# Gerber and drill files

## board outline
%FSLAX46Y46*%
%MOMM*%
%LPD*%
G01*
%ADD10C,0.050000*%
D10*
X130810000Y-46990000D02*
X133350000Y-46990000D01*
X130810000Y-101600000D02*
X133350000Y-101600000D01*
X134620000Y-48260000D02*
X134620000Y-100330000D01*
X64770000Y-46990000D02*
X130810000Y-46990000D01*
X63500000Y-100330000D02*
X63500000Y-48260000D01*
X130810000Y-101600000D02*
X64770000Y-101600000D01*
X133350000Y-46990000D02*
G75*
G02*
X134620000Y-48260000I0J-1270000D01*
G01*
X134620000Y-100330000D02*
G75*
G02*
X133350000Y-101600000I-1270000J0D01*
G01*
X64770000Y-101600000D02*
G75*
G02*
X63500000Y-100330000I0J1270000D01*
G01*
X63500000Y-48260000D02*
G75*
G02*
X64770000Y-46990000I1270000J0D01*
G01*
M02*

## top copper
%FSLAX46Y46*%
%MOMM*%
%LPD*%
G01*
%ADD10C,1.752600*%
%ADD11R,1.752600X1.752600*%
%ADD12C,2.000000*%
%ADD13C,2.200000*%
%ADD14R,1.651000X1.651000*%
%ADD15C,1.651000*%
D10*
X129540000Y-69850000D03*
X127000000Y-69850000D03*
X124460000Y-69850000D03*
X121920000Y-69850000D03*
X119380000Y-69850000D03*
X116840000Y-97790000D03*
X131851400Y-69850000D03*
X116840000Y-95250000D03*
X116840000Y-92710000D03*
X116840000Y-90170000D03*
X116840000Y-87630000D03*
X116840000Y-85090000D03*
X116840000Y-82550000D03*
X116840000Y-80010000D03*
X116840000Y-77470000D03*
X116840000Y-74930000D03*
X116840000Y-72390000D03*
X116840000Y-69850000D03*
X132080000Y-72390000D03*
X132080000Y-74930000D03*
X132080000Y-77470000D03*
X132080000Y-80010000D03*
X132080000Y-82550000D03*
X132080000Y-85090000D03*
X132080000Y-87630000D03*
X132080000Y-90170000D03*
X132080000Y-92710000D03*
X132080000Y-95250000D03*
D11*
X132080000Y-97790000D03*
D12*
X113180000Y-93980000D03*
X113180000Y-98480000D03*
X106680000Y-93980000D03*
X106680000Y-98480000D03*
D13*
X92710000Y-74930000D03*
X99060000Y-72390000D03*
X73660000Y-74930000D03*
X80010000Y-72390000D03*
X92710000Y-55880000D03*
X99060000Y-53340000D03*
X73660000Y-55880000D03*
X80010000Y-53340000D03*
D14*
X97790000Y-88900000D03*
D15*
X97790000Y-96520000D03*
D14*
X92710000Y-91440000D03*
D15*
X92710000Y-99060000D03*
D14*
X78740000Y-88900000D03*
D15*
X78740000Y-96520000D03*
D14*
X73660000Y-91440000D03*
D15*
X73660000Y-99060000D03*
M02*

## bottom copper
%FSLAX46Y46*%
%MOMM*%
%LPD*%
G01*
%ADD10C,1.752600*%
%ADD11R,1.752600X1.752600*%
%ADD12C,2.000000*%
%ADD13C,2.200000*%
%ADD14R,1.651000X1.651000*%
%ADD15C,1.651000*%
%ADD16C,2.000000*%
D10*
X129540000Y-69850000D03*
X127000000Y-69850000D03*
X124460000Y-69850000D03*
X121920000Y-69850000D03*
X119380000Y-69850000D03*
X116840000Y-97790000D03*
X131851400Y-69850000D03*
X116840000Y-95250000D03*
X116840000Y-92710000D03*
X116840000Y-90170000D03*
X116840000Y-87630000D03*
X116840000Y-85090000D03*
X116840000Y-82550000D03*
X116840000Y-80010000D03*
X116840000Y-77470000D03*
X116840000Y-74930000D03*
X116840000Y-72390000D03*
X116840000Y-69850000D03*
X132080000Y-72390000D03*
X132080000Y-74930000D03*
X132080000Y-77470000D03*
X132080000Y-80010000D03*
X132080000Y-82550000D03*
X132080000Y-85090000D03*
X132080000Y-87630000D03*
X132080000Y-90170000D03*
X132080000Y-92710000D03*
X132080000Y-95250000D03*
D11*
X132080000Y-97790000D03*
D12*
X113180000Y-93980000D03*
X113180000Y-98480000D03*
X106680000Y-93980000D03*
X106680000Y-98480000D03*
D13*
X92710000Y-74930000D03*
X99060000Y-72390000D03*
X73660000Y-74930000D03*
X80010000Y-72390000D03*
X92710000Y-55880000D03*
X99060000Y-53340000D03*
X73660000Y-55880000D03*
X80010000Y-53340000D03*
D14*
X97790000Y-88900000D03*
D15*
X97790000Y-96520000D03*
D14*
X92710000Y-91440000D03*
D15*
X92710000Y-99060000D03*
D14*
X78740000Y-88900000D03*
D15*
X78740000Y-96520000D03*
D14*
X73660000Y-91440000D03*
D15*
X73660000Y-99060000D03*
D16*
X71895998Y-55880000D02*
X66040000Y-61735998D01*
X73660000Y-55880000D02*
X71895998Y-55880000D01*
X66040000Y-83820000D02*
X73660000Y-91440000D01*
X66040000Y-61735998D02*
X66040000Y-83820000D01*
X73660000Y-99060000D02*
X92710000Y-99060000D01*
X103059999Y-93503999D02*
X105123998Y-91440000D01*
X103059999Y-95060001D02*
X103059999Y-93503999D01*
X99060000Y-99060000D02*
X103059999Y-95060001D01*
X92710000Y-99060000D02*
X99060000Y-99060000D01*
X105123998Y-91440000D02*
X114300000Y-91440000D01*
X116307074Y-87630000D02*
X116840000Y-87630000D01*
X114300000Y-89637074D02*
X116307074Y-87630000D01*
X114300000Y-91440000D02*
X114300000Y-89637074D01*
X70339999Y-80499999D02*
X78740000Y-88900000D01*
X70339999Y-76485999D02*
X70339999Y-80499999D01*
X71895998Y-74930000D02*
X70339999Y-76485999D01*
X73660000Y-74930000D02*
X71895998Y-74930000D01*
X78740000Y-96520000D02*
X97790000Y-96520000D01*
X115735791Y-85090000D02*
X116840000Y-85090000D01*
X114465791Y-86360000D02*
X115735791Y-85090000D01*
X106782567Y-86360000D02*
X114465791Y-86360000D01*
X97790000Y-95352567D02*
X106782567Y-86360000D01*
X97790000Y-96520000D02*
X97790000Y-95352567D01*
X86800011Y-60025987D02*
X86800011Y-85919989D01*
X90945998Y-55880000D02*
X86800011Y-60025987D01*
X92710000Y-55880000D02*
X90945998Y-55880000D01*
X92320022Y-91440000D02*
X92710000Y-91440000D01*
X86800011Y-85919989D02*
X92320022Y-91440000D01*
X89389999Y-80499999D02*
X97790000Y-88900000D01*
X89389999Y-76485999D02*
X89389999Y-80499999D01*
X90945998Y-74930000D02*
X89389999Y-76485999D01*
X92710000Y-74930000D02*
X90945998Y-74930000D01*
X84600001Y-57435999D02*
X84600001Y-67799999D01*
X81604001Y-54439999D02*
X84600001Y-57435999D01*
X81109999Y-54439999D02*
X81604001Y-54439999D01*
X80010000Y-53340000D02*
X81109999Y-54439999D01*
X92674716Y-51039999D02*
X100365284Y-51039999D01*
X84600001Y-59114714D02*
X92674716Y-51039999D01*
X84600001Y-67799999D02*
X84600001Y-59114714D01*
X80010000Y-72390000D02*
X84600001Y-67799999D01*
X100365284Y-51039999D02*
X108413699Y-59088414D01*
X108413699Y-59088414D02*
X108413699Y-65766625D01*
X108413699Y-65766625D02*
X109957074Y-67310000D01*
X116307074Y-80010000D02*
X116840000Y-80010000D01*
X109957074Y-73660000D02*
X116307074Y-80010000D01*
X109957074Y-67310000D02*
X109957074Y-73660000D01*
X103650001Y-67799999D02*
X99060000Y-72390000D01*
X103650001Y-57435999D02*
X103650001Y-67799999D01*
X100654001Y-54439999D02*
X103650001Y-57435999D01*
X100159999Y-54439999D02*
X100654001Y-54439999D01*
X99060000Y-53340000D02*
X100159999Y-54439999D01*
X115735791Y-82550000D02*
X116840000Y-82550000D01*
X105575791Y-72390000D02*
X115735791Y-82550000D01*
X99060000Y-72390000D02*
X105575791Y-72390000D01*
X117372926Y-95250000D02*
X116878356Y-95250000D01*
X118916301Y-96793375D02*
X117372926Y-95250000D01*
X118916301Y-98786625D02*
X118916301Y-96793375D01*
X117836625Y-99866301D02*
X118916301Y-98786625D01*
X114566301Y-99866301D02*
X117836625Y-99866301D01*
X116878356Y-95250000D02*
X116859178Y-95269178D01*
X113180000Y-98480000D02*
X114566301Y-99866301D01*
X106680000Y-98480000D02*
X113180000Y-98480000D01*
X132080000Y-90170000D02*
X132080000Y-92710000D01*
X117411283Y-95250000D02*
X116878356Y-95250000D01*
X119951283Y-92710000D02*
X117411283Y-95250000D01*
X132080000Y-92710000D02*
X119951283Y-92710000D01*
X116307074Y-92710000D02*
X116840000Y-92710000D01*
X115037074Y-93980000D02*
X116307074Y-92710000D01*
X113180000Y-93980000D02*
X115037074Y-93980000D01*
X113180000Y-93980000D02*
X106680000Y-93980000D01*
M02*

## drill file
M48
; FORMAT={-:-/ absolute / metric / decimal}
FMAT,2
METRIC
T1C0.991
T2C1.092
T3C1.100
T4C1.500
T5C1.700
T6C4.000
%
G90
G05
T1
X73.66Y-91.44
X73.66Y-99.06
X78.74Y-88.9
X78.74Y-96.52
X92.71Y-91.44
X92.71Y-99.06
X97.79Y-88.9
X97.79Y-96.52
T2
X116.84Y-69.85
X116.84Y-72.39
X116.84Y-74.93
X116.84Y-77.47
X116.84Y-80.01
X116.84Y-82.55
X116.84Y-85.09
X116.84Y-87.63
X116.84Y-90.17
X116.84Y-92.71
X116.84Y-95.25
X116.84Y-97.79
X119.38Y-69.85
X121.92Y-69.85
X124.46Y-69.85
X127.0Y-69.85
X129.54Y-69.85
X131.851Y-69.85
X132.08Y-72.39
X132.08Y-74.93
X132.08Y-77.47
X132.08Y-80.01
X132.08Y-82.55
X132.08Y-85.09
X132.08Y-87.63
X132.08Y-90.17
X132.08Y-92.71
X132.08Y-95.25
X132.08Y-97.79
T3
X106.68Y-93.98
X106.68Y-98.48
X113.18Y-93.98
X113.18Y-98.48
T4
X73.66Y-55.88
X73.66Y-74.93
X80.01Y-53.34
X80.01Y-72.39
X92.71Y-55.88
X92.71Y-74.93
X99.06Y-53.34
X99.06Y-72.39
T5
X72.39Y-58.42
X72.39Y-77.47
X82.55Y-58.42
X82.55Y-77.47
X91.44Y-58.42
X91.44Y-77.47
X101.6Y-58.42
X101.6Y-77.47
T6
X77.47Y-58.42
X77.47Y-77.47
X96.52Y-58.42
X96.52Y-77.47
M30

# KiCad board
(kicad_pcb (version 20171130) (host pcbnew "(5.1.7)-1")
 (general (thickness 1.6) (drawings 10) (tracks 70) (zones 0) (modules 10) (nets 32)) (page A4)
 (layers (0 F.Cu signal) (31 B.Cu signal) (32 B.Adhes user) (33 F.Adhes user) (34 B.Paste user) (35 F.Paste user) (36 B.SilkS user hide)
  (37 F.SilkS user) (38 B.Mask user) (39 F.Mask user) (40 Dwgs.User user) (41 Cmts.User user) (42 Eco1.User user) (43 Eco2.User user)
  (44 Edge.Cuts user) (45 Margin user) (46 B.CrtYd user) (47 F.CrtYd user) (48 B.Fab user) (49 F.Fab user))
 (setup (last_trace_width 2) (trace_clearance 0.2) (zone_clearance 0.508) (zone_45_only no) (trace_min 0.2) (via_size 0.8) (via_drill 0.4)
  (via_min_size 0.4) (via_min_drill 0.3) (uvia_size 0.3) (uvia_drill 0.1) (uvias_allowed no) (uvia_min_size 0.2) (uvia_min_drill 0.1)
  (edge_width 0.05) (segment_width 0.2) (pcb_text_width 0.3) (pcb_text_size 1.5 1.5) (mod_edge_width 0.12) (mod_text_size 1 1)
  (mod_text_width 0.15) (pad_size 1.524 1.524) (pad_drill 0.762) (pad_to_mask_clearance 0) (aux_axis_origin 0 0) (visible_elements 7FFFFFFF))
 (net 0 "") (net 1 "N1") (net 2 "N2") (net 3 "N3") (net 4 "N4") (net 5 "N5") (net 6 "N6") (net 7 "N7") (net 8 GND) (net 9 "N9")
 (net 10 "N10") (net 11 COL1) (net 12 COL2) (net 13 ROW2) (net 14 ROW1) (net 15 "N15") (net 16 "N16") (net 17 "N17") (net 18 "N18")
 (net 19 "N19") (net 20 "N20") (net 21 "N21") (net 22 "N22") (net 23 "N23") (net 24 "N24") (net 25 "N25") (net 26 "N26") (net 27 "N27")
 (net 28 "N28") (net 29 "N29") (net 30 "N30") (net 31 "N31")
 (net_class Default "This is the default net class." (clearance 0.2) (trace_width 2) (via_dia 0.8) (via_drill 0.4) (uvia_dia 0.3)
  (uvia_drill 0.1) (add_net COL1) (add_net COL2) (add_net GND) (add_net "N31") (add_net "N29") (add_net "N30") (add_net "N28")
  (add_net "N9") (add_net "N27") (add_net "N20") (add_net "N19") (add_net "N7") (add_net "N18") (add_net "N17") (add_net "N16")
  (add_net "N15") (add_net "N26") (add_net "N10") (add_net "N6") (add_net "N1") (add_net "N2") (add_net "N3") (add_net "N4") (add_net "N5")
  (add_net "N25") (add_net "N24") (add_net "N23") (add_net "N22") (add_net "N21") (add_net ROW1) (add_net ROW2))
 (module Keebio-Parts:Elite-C (layer F.Cu) (at 124.46 83.82 90)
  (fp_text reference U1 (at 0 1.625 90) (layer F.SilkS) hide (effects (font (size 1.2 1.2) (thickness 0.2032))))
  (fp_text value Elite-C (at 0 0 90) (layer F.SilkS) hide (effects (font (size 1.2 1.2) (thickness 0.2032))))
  (pad 25 thru_hole circle (at 13.97 5.08 90) (size 1.7526 1.7526) (drill 1.0922) (layers *.Cu *.SilkS *.Mask) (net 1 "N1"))
  (pad 26 thru_hole circle (at 13.97 2.54 90) (size 1.7526 1.7526) (drill 1.0922) (layers *.Cu *.SilkS *.Mask) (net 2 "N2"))
  (pad 27 thru_hole circle (at 13.97 0 90) (size 1.7526 1.7526) (drill 1.0922) (layers *.Cu *.SilkS *.Mask) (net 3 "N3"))
  (pad 28 thru_hole circle (at 13.97 -2.54 90) (size 1.7526 1.7526) (drill 1.0922) (layers *.Cu *.SilkS *.Mask) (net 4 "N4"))
  (pad 29 thru_hole circle (at 13.97 -5.08 90) (size 1.7526 1.7526) (drill 1.0922) (layers *.Cu *.SilkS *.Mask) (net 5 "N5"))
  (pad 24 thru_hole circle (at -13.97 -7.62 90) (size 1.7526 1.7526) (drill 1.0922) (layers *.Cu *.SilkS *.Mask) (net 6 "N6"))
  (pad 12 thru_hole circle (at 13.97 7.3914 90) (size 1.7526 1.7526) (drill 1.0922) (layers *.Cu *.SilkS *.Mask) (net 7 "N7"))
  (pad 23 thru_hole circle (at -11.43 -7.62 90) (size 1.7526 1.7526) (drill 1.0922) (layers *.Cu *.SilkS *.Mask) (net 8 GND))
  (pad 22 thru_hole circle (at -8.89 -7.62 90) (size 1.7526 1.7526) (drill 1.0922) (layers *.Cu *.SilkS *.Mask) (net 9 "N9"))
  (pad 21 thru_hole circle (at -6.35 -7.62 90) (size 1.7526 1.7526) (drill 1.0922) (layers *.Cu *.SilkS *.Mask) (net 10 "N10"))
  (pad 20 thru_hole circle (at -3.81 -7.62 90) (size 1.7526 1.7526) (drill 1.0922) (layers *.Cu *.SilkS *.Mask) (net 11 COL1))
  (pad 19 thru_hole circle (at -1.27 -7.62 90) (size 1.7526 1.7526) (drill 1.0922) (layers *.Cu *.SilkS *.Mask) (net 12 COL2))
  (pad 18 thru_hole circle (at 1.27 -7.62 90) (size 1.7526 1.7526) (drill 1.0922) (layers *.Cu *.SilkS *.Mask) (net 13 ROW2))
  (pad 17 thru_hole circle (at 3.81 -7.62 90) (size 1.7526 1.7526) (drill 1.0922) (layers *.Cu *.SilkS *.Mask) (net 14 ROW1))
  (pad 16 thru_hole circle (at 6.35 -7.62 90) (size 1.7526 1.7526) (drill 1.0922) (layers *.Cu *.SilkS *.Mask) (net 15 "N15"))
  (pad 15 thru_hole circle (at 8.89 -7.62 90) (size 1.7526 1.7526) (drill 1.0922) (layers *.Cu *.SilkS *.Mask) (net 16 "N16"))
  (pad 14 thru_hole circle (at 11.43 -7.62 90) (size 1.7526 1.7526) (drill 1.0922) (layers *.Cu *.SilkS *.Mask) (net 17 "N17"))
  (pad 13 thru_hole circle (at 13.97 -7.62 90) (size 1.7526 1.7526) (drill 1.0922) (layers *.Cu *.SilkS *.Mask) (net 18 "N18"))
  (pad 11 thru_hole circle (at 11.43 7.62 90) (size 1.7526 1.7526) (drill 1.0922) (layers *.Cu *.SilkS *.Mask) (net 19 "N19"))
  (pad 10 thru_hole circle (at 8.89 7.62 90) (size 1.7526 1.7526) (drill 1.0922) (layers *.Cu *.SilkS *.Mask) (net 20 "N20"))
  (pad 9 thru_hole circle (at 6.35 7.62 90) (size 1.7526 1.7526) (drill 1.0922) (layers *.Cu *.SilkS *.Mask) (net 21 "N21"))
  (pad 8 thru_hole circle (at 3.81 7.62 90) (size 1.7526 1.7526) (drill 1.0922) (layers *.Cu *.SilkS *.Mask) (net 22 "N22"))
  (pad 7 thru_hole circle (at 1.27 7.62 90) (size 1.7526 1.7526) (drill 1.0922) (layers *.Cu *.SilkS *.Mask) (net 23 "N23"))
  (pad 6 thru_hole circle (at -1.27 7.62 90) (size 1.7526 1.7526) (drill 1.0922) (layers *.Cu *.SilkS *.Mask) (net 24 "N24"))
  (pad 5 thru_hole circle (at -3.81 7.62 90) (size 1.7526 1.7526) (drill 1.0922) (layers *.Cu *.SilkS *.Mask) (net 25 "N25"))
  (pad 4 thru_hole circle (at -6.35 7.62 90) (size 1.7526 1.7526) (drill 1.0922) (layers *.Cu *.SilkS *.Mask) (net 8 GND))
  (pad 3 thru_hole circle (at -8.89 7.62 90) (size 1.7526 1.7526) (drill 1.0922) (layers *.Cu *.SilkS *.Mask) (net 8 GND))
  (pad 2 thru_hole circle (at -11.43 7.62 90) (size 1.7526 1.7526) (drill 1.0922) (layers *.Cu *.SilkS *.Mask) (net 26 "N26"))
  (pad 1 thru_hole rect (at -13.97 7.62 90) (size 1.7526 1.7526) (drill 1.0922) (layers *.Cu *.SilkS *.Mask) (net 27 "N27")))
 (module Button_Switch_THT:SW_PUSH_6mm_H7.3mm (layer F.Cu) (at 106.68 93.98)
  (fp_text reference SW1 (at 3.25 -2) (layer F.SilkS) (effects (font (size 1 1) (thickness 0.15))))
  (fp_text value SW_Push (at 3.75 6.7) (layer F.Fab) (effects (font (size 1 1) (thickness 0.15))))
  (pad 1 thru_hole circle (at 6.5 0 90) (size 2 2) (drill 1.1) (layers *.Cu *.Mask) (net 9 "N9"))
  (pad 2 thru_hole circle (at 6.5 4.5 90) (size 2 2) (drill 1.1) (layers *.Cu *.Mask) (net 8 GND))
  (pad 1 thru_hole circle (at 0 0 90) (size 2 2) (drill 1.1) (layers *.Cu *.Mask) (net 9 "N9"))
  (pad 2 thru_hole circle (at 0 4.5 90) (size 2 2) (drill 1.1) (layers *.Cu *.Mask) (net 8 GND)))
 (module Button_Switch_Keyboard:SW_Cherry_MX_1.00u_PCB (layer F.Cu) (at 99.06 72.39)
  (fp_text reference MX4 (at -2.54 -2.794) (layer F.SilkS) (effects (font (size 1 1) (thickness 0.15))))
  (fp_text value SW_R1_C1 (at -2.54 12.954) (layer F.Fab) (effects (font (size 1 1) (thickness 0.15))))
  (pad "" np_thru_hole circle (at 2.54 5.08) (size 1.7 1.7) (drill 1.7) (layers *.Cu *.Mask))
  (pad "" np_thru_hole circle (at -7.62 5.08) (size 1.7 1.7) (drill 1.7) (layers *.Cu *.Mask))
  (pad "" np_thru_hole circle (at -2.54 5.08) (size 4 4) (drill 4) (layers *.Cu *.Mask))
  (pad 2 thru_hole circle (at -6.35 2.54) (size 2.2 2.2) (drill 1.5) (layers *.Cu *.Mask) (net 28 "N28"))
  (pad 1 thru_hole circle (at 0 0) (size 2.2 2.2) (drill 1.5) (layers *.Cu *.Mask) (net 13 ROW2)))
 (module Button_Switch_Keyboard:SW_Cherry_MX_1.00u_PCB (layer F.Cu) (at 80.01 72.39)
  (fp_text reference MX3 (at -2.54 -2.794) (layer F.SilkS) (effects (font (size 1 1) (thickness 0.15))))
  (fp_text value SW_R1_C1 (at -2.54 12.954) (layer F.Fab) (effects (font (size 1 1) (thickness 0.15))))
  (pad "" np_thru_hole circle (at 2.54 5.08) (size 1.7 1.7) (drill 1.7) (layers *.Cu *.Mask))
  (pad "" np_thru_hole circle (at -7.62 5.08) (size 1.7 1.7) (drill 1.7) (layers *.Cu *.Mask))
  (pad "" np_thru_hole circle (at -2.54 5.08) (size 4 4) (drill 4) (layers *.Cu *.Mask))
  (pad 2 thru_hole circle (at -6.35 2.54) (size 2.2 2.2) (drill 1.5) (layers *.Cu *.Mask) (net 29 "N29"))
  (pad 1 thru_hole circle (at 0 0) (size 2.2 2.2) (drill 1.5) (layers *.Cu *.Mask) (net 14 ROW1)))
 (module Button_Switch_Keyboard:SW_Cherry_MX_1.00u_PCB (layer F.Cu) (at 99.06 53.34)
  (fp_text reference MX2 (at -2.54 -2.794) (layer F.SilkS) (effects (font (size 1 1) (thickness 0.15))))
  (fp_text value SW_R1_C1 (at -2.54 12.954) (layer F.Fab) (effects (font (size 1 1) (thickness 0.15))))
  (pad "" np_thru_hole circle (at 2.54 5.08) (size 1.7 1.7) (drill 1.7) (layers *.Cu *.Mask))
  (pad "" np_thru_hole circle (at -7.62 5.08) (size 1.7 1.7) (drill 1.7) (layers *.Cu *.Mask))
  (pad "" np_thru_hole circle (at -2.54 5.08) (size 4 4) (drill 4) (layers *.Cu *.Mask))
  (pad 2 thru_hole circle (at -6.35 2.54) (size 2.2 2.2) (drill 1.5) (layers *.Cu *.Mask) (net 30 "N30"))
  (pad 1 thru_hole circle (at 0 0) (size 2.2 2.2) (drill 1.5) (layers *.Cu *.Mask) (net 13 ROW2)))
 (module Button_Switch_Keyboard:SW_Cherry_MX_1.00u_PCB (layer F.Cu) (at 80.01 53.34)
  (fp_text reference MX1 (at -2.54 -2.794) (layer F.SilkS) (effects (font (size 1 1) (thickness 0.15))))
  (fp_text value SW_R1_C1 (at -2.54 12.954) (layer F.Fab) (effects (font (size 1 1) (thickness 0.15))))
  (pad "" np_thru_hole circle (at 2.54 5.08) (size 1.7 1.7) (drill 1.7) (layers *.Cu *.Mask))
  (pad "" np_thru_hole circle (at -7.62 5.08) (size 1.7 1.7) (drill 1.7) (layers *.Cu *.Mask))
  (pad "" np_thru_hole circle (at -2.54 5.08) (size 4 4) (drill 4) (layers *.Cu *.Mask))
  (pad 2 thru_hole circle (at -6.35 2.54) (size 2.2 2.2) (drill 1.5) (layers *.Cu *.Mask) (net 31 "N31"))
  (pad 1 thru_hole circle (at 0 0) (size 2.2 2.2) (drill 1.5) (layers *.Cu *.Mask) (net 14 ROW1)))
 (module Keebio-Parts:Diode (layer F.Cu) (at 97.79 92.71 90)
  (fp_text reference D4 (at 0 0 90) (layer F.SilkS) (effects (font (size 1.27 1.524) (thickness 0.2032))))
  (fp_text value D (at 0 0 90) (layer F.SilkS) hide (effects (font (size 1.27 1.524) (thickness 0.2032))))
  (pad 2 thru_hole rect (at 3.81 0 90) (size 1.651 1.651) (drill 0.9906) (layers *.Cu *.SilkS *.Mask) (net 28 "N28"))
  (pad 1 thru_hole circle (at -3.81 0 90) (size 1.651 1.651) (drill 0.9906) (layers *.Cu *.SilkS *.Mask) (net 12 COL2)))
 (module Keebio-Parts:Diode (layer F.Cu) (at 92.71 95.25 90)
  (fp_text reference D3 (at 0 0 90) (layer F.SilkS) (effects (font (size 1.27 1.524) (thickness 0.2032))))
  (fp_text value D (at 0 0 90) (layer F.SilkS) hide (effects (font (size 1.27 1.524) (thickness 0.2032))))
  (pad 2 thru_hole rect (at 3.81 0 90) (size 1.651 1.651) (drill 0.9906) (layers *.Cu *.SilkS *.Mask) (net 30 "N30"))
  (pad 1 thru_hole circle (at -3.81 0 90) (size 1.651 1.651) (drill 0.9906) (layers *.Cu *.SilkS *.Mask) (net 11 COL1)))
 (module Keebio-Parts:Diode (layer F.Cu) (at 78.74 92.71 90)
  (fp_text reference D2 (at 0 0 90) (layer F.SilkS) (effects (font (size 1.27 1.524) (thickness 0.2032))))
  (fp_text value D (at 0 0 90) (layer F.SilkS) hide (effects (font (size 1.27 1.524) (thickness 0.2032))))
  (pad 2 thru_hole rect (at 3.81 0 90) (size 1.651 1.651) (drill 0.9906) (layers *.Cu *.SilkS *.Mask) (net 29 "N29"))
  (pad 1 thru_hole circle (at -3.81 0 90) (size 1.651 1.651) (drill 0.9906) (layers *.Cu *.SilkS *.Mask) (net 12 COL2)))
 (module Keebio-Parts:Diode (layer F.Cu) (at 73.66 95.25 90)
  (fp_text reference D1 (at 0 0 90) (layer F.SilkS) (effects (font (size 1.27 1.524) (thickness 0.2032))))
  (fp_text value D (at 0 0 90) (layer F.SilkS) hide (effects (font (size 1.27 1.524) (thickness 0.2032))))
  (pad 2 thru_hole rect (at 3.81 0 90) (size 1.651 1.651) (drill 0.9906) (layers *.Cu *.SilkS *.Mask) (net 31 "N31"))
  (pad 1 thru_hole circle (at -3.81 0 90) (size 1.651 1.651) (drill 0.9906) (layers *.Cu *.SilkS *.Mask) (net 11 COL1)))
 (gr_line (start 130.81 46.99) (end 133.35 46.99) (layer Edge.Cuts) (width 0.05))
 (gr_line (start 130.81 101.6) (end 133.35 101.6) (layer Edge.Cuts) (width 0.05))
 (gr_line (start 134.62 48.26) (end 134.62 100.33) (layer Edge.Cuts) (width 0.05))
 (gr_line (start 64.77 46.99) (end 130.81 46.99) (layer Edge.Cuts) (width 0.05))
 (gr_line (start 63.5 100.33) (end 63.5 48.26) (layer Edge.Cuts) (width 0.05))
 (gr_line (start 130.81 101.6) (end 64.77 101.6) (layer Edge.Cuts) (width 0.05))
 (gr_arc (start 133.35 48.26) (end 134.62 48.26) (angle -90) (layer Edge.Cuts) (width 0.05))
 (gr_arc (start 133.35 100.33) (end 133.35 101.6) (angle -90) (layer Edge.Cuts) (width 0.05))
 (gr_arc (start 64.77 100.33) (end 63.5 100.33) (angle -90) (layer Edge.Cuts) (width 0.05))
 (gr_arc (start 64.77 48.26) (end 64.77 46.99) (angle -90) (layer Edge.Cuts) (width 0.05))
 (segment (start 71.895998 55.88) (end 66.04 61.735998) (width 2) (layer B.Cu) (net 31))
 (segment (start 73.66 55.88) (end 71.895998 55.88) (width 2) (layer B.Cu) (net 31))
 (segment (start 66.04 83.82) (end 73.66 91.44) (width 2) (layer B.Cu) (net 31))
 (segment (start 66.04 61.735998) (end 66.04 83.82) (width 2) (layer B.Cu) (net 31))
 (segment (start 73.66 99.06) (end 92.71 99.06) (width 2) (layer B.Cu) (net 11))
 (segment (start 103.059999 93.503999) (end 105.123998 91.44) (width 2) (layer B.Cu) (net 11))
 (segment (start 103.059999 95.060001) (end 103.059999 93.503999) (width 2) (layer B.Cu) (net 11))
 (segment (start 99.06 99.06) (end 103.059999 95.060001) (width 2) (layer B.Cu) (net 11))
 (segment (start 92.71 99.06) (end 99.06 99.06) (width 2) (layer B.Cu) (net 11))
 (segment (start 105.123998 91.44) (end 114.3 91.44) (width 2) (layer B.Cu) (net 11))
 (segment (start 116.307074 87.63) (end 116.84 87.63) (width 2) (layer B.Cu) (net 11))
 (segment (start 114.3 89.637074) (end 116.307074 87.63) (width 2) (layer B.Cu) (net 11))
 (segment (start 114.3 91.44) (end 114.3 89.637074) (width 2) (layer B.Cu) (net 11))
 (segment (start 70.339999 80.499999) (end 78.74 88.9) (width 2) (layer B.Cu) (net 29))
 (segment (start 70.339999 76.485999) (end 70.339999 80.499999) (width 2) (layer B.Cu) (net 29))
 (segment (start 71.895998 74.93) (end 70.339999 76.485999) (width 2) (layer B.Cu) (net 29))
 (segment (start 73.66 74.93) (end 71.895998 74.93) (width 2) (layer B.Cu) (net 29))
 (segment (start 78.74 96.52) (end 97.79 96.52) (width 2) (layer B.Cu) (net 12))
 (segment (start 115.735791 85.09) (end 116.84 85.09) (width 2) (layer B.Cu) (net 12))
 (segment (start 114.465791 86.36) (end 115.735791 85.09) (width 2) (layer B.Cu) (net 12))
 (segment (start 106.782567 86.36) (end 114.465791 86.36) (width 2) (layer B.Cu) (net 12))
 (segment (start 97.79 95.352567) (end 106.782567 86.36) (width 2) (layer B.Cu) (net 12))
 (segment (start 97.79 96.52) (end 97.79 95.352567) (width 2) (layer B.Cu) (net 12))
 (segment (start 86.800011 60.025987) (end 86.800011 85.919989) (width 2) (layer B.Cu) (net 30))
 (segment (start 90.945998 55.88) (end 86.800011 60.025987) (width 2) (layer B.Cu) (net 30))
 (segment (start 92.71 55.88) (end 90.945998 55.88) (width 2) (layer B.Cu) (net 30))
 (segment (start 92.320022 91.44) (end 92.71 91.44) (width 2) (layer B.Cu) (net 30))
 (segment (start 86.800011 85.919989) (end 92.320022 91.44) (width 2) (layer B.Cu) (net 30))
 (segment (start 89.389999 80.499999) (end 97.79 88.9) (width 2) (layer B.Cu) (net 28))
 (segment (start 89.389999 76.485999) (end 89.389999 80.499999) (width 2) (layer B.Cu) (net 28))
 (segment (start 90.945998 74.93) (end 89.389999 76.485999) (width 2) (layer B.Cu) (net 28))
 (segment (start 92.71 74.93) (end 90.945998 74.93) (width 2) (layer B.Cu) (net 28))
 (segment (start 84.600001 57.435999) (end 84.600001 67.799999) (width 2) (layer B.Cu) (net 14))
 (segment (start 81.604001 54.439999) (end 84.600001 57.435999) (width 2) (layer B.Cu) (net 14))
 (segment (start 81.109999 54.439999) (end 81.604001 54.439999) (width 2) (layer B.Cu) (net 14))
 (segment (start 80.01 53.34) (end 81.109999 54.439999) (width 2) (layer B.Cu) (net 14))
 (segment (start 92.674716 51.039999) (end 100.365284 51.039999) (width 2) (layer B.Cu) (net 14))
 (segment (start 84.600001 59.114714) (end 92.674716 51.039999) (width 2) (layer B.Cu) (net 14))
 (segment (start 84.600001 67.799999) (end 84.600001 59.114714) (width 2) (layer B.Cu) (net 14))
 (segment (start 80.01 72.39) (end 84.600001 67.799999) (width 2) (layer B.Cu) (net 14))
 (segment (start 100.365284 51.039999) (end 108.413699 59.088414) (width 2) (layer B.Cu) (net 14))
 (segment (start 108.413699 59.088414) (end 108.413699 65.766625) (width 2) (layer B.Cu) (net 14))
 (segment (start 108.413699 65.766625) (end 109.957074 67.31) (width 2) (layer B.Cu) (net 14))
 (segment (start 116.307074 80.01) (end 116.84 80.01) (width 2) (layer B.Cu) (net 14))
 (segment (start 109.957074 73.66) (end 116.307074 80.01) (width 2) (layer B.Cu) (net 14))
 (segment (start 109.957074 67.31) (end 109.957074 73.66) (width 2) (layer B.Cu) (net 14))
 (segment (start 103.650001 67.799999) (end 99.06 72.39) (width 2) (layer B.Cu) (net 13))
 (segment (start 103.650001 57.435999) (end 103.650001 67.799999) (width 2) (layer B.Cu) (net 13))
 (segment (start 100.654001 54.439999) (end 103.650001 57.435999) (width 2) (layer B.Cu) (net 13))
 (segment (start 100.159999 54.439999) (end 100.654001 54.439999) (width 2) (layer B.Cu) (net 13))
 (segment (start 99.06 53.34) (end 100.159999 54.439999) (width 2) (layer B.Cu) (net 13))
 (segment (start 115.735791 82.55) (end 116.84 82.55) (width 2) (layer B.Cu) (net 13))
 (segment (start 105.575791 72.39) (end 115.735791 82.55) (width 2) (layer B.Cu) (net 13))
 (segment (start 99.06 72.39) (end 105.575791 72.39) (width 2) (layer B.Cu) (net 13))
 (segment (start 117.372926 95.25) (end 116.878356 95.25) (width 2) (layer B.Cu) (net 8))
 (segment (start 118.916301 96.793375) (end 117.372926 95.25) (width 2) (layer B.Cu) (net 8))
 (segment (start 118.916301 98.786625) (end 118.916301 96.793375) (width 2) (layer B.Cu) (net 8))
 (segment (start 117.836625 99.866301) (end 118.916301 98.786625) (width 2) (layer B.Cu) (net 8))
 (segment (start 114.566301 99.866301) (end 117.836625 99.866301) (width 2) (layer B.Cu) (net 8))
 (segment (start 116.878356 95.25) (end 116.859178 95.269178) (width 2) (layer B.Cu) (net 8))
 (segment (start 113.18 98.48) (end 114.566301 99.866301) (width 2) (layer B.Cu) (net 8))
 (segment (start 106.68 98.48) (end 113.18 98.48) (width 2) (layer B.Cu) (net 8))
 (segment (start 132.08 90.17) (end 132.08 92.71) (width 2) (layer B.Cu) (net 8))
 (segment (start 117.411283 95.25) (end 116.878356 95.25) (width 2) (layer B.Cu) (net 8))
 (segment (start 119.951283 92.71) (end 117.411283 95.25) (width 2) (layer B.Cu) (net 8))
 (segment (start 132.08 92.71) (end 119.951283 92.71) (width 2) (layer B.Cu) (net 8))
 (segment (start 116.307074 92.71) (end 116.84 92.71) (width 2) (layer B.Cu) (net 9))
 (segment (start 115.037074 93.98) (end 116.307074 92.71) (width 2) (layer B.Cu) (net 9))
 (segment (start 113.18 93.98) (end 115.037074 93.98) (width 2) (layer B.Cu) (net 9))
 (segment (start 113.18 93.98) (end 106.68 93.98) (width 2) (layer B.Cu) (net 9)))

